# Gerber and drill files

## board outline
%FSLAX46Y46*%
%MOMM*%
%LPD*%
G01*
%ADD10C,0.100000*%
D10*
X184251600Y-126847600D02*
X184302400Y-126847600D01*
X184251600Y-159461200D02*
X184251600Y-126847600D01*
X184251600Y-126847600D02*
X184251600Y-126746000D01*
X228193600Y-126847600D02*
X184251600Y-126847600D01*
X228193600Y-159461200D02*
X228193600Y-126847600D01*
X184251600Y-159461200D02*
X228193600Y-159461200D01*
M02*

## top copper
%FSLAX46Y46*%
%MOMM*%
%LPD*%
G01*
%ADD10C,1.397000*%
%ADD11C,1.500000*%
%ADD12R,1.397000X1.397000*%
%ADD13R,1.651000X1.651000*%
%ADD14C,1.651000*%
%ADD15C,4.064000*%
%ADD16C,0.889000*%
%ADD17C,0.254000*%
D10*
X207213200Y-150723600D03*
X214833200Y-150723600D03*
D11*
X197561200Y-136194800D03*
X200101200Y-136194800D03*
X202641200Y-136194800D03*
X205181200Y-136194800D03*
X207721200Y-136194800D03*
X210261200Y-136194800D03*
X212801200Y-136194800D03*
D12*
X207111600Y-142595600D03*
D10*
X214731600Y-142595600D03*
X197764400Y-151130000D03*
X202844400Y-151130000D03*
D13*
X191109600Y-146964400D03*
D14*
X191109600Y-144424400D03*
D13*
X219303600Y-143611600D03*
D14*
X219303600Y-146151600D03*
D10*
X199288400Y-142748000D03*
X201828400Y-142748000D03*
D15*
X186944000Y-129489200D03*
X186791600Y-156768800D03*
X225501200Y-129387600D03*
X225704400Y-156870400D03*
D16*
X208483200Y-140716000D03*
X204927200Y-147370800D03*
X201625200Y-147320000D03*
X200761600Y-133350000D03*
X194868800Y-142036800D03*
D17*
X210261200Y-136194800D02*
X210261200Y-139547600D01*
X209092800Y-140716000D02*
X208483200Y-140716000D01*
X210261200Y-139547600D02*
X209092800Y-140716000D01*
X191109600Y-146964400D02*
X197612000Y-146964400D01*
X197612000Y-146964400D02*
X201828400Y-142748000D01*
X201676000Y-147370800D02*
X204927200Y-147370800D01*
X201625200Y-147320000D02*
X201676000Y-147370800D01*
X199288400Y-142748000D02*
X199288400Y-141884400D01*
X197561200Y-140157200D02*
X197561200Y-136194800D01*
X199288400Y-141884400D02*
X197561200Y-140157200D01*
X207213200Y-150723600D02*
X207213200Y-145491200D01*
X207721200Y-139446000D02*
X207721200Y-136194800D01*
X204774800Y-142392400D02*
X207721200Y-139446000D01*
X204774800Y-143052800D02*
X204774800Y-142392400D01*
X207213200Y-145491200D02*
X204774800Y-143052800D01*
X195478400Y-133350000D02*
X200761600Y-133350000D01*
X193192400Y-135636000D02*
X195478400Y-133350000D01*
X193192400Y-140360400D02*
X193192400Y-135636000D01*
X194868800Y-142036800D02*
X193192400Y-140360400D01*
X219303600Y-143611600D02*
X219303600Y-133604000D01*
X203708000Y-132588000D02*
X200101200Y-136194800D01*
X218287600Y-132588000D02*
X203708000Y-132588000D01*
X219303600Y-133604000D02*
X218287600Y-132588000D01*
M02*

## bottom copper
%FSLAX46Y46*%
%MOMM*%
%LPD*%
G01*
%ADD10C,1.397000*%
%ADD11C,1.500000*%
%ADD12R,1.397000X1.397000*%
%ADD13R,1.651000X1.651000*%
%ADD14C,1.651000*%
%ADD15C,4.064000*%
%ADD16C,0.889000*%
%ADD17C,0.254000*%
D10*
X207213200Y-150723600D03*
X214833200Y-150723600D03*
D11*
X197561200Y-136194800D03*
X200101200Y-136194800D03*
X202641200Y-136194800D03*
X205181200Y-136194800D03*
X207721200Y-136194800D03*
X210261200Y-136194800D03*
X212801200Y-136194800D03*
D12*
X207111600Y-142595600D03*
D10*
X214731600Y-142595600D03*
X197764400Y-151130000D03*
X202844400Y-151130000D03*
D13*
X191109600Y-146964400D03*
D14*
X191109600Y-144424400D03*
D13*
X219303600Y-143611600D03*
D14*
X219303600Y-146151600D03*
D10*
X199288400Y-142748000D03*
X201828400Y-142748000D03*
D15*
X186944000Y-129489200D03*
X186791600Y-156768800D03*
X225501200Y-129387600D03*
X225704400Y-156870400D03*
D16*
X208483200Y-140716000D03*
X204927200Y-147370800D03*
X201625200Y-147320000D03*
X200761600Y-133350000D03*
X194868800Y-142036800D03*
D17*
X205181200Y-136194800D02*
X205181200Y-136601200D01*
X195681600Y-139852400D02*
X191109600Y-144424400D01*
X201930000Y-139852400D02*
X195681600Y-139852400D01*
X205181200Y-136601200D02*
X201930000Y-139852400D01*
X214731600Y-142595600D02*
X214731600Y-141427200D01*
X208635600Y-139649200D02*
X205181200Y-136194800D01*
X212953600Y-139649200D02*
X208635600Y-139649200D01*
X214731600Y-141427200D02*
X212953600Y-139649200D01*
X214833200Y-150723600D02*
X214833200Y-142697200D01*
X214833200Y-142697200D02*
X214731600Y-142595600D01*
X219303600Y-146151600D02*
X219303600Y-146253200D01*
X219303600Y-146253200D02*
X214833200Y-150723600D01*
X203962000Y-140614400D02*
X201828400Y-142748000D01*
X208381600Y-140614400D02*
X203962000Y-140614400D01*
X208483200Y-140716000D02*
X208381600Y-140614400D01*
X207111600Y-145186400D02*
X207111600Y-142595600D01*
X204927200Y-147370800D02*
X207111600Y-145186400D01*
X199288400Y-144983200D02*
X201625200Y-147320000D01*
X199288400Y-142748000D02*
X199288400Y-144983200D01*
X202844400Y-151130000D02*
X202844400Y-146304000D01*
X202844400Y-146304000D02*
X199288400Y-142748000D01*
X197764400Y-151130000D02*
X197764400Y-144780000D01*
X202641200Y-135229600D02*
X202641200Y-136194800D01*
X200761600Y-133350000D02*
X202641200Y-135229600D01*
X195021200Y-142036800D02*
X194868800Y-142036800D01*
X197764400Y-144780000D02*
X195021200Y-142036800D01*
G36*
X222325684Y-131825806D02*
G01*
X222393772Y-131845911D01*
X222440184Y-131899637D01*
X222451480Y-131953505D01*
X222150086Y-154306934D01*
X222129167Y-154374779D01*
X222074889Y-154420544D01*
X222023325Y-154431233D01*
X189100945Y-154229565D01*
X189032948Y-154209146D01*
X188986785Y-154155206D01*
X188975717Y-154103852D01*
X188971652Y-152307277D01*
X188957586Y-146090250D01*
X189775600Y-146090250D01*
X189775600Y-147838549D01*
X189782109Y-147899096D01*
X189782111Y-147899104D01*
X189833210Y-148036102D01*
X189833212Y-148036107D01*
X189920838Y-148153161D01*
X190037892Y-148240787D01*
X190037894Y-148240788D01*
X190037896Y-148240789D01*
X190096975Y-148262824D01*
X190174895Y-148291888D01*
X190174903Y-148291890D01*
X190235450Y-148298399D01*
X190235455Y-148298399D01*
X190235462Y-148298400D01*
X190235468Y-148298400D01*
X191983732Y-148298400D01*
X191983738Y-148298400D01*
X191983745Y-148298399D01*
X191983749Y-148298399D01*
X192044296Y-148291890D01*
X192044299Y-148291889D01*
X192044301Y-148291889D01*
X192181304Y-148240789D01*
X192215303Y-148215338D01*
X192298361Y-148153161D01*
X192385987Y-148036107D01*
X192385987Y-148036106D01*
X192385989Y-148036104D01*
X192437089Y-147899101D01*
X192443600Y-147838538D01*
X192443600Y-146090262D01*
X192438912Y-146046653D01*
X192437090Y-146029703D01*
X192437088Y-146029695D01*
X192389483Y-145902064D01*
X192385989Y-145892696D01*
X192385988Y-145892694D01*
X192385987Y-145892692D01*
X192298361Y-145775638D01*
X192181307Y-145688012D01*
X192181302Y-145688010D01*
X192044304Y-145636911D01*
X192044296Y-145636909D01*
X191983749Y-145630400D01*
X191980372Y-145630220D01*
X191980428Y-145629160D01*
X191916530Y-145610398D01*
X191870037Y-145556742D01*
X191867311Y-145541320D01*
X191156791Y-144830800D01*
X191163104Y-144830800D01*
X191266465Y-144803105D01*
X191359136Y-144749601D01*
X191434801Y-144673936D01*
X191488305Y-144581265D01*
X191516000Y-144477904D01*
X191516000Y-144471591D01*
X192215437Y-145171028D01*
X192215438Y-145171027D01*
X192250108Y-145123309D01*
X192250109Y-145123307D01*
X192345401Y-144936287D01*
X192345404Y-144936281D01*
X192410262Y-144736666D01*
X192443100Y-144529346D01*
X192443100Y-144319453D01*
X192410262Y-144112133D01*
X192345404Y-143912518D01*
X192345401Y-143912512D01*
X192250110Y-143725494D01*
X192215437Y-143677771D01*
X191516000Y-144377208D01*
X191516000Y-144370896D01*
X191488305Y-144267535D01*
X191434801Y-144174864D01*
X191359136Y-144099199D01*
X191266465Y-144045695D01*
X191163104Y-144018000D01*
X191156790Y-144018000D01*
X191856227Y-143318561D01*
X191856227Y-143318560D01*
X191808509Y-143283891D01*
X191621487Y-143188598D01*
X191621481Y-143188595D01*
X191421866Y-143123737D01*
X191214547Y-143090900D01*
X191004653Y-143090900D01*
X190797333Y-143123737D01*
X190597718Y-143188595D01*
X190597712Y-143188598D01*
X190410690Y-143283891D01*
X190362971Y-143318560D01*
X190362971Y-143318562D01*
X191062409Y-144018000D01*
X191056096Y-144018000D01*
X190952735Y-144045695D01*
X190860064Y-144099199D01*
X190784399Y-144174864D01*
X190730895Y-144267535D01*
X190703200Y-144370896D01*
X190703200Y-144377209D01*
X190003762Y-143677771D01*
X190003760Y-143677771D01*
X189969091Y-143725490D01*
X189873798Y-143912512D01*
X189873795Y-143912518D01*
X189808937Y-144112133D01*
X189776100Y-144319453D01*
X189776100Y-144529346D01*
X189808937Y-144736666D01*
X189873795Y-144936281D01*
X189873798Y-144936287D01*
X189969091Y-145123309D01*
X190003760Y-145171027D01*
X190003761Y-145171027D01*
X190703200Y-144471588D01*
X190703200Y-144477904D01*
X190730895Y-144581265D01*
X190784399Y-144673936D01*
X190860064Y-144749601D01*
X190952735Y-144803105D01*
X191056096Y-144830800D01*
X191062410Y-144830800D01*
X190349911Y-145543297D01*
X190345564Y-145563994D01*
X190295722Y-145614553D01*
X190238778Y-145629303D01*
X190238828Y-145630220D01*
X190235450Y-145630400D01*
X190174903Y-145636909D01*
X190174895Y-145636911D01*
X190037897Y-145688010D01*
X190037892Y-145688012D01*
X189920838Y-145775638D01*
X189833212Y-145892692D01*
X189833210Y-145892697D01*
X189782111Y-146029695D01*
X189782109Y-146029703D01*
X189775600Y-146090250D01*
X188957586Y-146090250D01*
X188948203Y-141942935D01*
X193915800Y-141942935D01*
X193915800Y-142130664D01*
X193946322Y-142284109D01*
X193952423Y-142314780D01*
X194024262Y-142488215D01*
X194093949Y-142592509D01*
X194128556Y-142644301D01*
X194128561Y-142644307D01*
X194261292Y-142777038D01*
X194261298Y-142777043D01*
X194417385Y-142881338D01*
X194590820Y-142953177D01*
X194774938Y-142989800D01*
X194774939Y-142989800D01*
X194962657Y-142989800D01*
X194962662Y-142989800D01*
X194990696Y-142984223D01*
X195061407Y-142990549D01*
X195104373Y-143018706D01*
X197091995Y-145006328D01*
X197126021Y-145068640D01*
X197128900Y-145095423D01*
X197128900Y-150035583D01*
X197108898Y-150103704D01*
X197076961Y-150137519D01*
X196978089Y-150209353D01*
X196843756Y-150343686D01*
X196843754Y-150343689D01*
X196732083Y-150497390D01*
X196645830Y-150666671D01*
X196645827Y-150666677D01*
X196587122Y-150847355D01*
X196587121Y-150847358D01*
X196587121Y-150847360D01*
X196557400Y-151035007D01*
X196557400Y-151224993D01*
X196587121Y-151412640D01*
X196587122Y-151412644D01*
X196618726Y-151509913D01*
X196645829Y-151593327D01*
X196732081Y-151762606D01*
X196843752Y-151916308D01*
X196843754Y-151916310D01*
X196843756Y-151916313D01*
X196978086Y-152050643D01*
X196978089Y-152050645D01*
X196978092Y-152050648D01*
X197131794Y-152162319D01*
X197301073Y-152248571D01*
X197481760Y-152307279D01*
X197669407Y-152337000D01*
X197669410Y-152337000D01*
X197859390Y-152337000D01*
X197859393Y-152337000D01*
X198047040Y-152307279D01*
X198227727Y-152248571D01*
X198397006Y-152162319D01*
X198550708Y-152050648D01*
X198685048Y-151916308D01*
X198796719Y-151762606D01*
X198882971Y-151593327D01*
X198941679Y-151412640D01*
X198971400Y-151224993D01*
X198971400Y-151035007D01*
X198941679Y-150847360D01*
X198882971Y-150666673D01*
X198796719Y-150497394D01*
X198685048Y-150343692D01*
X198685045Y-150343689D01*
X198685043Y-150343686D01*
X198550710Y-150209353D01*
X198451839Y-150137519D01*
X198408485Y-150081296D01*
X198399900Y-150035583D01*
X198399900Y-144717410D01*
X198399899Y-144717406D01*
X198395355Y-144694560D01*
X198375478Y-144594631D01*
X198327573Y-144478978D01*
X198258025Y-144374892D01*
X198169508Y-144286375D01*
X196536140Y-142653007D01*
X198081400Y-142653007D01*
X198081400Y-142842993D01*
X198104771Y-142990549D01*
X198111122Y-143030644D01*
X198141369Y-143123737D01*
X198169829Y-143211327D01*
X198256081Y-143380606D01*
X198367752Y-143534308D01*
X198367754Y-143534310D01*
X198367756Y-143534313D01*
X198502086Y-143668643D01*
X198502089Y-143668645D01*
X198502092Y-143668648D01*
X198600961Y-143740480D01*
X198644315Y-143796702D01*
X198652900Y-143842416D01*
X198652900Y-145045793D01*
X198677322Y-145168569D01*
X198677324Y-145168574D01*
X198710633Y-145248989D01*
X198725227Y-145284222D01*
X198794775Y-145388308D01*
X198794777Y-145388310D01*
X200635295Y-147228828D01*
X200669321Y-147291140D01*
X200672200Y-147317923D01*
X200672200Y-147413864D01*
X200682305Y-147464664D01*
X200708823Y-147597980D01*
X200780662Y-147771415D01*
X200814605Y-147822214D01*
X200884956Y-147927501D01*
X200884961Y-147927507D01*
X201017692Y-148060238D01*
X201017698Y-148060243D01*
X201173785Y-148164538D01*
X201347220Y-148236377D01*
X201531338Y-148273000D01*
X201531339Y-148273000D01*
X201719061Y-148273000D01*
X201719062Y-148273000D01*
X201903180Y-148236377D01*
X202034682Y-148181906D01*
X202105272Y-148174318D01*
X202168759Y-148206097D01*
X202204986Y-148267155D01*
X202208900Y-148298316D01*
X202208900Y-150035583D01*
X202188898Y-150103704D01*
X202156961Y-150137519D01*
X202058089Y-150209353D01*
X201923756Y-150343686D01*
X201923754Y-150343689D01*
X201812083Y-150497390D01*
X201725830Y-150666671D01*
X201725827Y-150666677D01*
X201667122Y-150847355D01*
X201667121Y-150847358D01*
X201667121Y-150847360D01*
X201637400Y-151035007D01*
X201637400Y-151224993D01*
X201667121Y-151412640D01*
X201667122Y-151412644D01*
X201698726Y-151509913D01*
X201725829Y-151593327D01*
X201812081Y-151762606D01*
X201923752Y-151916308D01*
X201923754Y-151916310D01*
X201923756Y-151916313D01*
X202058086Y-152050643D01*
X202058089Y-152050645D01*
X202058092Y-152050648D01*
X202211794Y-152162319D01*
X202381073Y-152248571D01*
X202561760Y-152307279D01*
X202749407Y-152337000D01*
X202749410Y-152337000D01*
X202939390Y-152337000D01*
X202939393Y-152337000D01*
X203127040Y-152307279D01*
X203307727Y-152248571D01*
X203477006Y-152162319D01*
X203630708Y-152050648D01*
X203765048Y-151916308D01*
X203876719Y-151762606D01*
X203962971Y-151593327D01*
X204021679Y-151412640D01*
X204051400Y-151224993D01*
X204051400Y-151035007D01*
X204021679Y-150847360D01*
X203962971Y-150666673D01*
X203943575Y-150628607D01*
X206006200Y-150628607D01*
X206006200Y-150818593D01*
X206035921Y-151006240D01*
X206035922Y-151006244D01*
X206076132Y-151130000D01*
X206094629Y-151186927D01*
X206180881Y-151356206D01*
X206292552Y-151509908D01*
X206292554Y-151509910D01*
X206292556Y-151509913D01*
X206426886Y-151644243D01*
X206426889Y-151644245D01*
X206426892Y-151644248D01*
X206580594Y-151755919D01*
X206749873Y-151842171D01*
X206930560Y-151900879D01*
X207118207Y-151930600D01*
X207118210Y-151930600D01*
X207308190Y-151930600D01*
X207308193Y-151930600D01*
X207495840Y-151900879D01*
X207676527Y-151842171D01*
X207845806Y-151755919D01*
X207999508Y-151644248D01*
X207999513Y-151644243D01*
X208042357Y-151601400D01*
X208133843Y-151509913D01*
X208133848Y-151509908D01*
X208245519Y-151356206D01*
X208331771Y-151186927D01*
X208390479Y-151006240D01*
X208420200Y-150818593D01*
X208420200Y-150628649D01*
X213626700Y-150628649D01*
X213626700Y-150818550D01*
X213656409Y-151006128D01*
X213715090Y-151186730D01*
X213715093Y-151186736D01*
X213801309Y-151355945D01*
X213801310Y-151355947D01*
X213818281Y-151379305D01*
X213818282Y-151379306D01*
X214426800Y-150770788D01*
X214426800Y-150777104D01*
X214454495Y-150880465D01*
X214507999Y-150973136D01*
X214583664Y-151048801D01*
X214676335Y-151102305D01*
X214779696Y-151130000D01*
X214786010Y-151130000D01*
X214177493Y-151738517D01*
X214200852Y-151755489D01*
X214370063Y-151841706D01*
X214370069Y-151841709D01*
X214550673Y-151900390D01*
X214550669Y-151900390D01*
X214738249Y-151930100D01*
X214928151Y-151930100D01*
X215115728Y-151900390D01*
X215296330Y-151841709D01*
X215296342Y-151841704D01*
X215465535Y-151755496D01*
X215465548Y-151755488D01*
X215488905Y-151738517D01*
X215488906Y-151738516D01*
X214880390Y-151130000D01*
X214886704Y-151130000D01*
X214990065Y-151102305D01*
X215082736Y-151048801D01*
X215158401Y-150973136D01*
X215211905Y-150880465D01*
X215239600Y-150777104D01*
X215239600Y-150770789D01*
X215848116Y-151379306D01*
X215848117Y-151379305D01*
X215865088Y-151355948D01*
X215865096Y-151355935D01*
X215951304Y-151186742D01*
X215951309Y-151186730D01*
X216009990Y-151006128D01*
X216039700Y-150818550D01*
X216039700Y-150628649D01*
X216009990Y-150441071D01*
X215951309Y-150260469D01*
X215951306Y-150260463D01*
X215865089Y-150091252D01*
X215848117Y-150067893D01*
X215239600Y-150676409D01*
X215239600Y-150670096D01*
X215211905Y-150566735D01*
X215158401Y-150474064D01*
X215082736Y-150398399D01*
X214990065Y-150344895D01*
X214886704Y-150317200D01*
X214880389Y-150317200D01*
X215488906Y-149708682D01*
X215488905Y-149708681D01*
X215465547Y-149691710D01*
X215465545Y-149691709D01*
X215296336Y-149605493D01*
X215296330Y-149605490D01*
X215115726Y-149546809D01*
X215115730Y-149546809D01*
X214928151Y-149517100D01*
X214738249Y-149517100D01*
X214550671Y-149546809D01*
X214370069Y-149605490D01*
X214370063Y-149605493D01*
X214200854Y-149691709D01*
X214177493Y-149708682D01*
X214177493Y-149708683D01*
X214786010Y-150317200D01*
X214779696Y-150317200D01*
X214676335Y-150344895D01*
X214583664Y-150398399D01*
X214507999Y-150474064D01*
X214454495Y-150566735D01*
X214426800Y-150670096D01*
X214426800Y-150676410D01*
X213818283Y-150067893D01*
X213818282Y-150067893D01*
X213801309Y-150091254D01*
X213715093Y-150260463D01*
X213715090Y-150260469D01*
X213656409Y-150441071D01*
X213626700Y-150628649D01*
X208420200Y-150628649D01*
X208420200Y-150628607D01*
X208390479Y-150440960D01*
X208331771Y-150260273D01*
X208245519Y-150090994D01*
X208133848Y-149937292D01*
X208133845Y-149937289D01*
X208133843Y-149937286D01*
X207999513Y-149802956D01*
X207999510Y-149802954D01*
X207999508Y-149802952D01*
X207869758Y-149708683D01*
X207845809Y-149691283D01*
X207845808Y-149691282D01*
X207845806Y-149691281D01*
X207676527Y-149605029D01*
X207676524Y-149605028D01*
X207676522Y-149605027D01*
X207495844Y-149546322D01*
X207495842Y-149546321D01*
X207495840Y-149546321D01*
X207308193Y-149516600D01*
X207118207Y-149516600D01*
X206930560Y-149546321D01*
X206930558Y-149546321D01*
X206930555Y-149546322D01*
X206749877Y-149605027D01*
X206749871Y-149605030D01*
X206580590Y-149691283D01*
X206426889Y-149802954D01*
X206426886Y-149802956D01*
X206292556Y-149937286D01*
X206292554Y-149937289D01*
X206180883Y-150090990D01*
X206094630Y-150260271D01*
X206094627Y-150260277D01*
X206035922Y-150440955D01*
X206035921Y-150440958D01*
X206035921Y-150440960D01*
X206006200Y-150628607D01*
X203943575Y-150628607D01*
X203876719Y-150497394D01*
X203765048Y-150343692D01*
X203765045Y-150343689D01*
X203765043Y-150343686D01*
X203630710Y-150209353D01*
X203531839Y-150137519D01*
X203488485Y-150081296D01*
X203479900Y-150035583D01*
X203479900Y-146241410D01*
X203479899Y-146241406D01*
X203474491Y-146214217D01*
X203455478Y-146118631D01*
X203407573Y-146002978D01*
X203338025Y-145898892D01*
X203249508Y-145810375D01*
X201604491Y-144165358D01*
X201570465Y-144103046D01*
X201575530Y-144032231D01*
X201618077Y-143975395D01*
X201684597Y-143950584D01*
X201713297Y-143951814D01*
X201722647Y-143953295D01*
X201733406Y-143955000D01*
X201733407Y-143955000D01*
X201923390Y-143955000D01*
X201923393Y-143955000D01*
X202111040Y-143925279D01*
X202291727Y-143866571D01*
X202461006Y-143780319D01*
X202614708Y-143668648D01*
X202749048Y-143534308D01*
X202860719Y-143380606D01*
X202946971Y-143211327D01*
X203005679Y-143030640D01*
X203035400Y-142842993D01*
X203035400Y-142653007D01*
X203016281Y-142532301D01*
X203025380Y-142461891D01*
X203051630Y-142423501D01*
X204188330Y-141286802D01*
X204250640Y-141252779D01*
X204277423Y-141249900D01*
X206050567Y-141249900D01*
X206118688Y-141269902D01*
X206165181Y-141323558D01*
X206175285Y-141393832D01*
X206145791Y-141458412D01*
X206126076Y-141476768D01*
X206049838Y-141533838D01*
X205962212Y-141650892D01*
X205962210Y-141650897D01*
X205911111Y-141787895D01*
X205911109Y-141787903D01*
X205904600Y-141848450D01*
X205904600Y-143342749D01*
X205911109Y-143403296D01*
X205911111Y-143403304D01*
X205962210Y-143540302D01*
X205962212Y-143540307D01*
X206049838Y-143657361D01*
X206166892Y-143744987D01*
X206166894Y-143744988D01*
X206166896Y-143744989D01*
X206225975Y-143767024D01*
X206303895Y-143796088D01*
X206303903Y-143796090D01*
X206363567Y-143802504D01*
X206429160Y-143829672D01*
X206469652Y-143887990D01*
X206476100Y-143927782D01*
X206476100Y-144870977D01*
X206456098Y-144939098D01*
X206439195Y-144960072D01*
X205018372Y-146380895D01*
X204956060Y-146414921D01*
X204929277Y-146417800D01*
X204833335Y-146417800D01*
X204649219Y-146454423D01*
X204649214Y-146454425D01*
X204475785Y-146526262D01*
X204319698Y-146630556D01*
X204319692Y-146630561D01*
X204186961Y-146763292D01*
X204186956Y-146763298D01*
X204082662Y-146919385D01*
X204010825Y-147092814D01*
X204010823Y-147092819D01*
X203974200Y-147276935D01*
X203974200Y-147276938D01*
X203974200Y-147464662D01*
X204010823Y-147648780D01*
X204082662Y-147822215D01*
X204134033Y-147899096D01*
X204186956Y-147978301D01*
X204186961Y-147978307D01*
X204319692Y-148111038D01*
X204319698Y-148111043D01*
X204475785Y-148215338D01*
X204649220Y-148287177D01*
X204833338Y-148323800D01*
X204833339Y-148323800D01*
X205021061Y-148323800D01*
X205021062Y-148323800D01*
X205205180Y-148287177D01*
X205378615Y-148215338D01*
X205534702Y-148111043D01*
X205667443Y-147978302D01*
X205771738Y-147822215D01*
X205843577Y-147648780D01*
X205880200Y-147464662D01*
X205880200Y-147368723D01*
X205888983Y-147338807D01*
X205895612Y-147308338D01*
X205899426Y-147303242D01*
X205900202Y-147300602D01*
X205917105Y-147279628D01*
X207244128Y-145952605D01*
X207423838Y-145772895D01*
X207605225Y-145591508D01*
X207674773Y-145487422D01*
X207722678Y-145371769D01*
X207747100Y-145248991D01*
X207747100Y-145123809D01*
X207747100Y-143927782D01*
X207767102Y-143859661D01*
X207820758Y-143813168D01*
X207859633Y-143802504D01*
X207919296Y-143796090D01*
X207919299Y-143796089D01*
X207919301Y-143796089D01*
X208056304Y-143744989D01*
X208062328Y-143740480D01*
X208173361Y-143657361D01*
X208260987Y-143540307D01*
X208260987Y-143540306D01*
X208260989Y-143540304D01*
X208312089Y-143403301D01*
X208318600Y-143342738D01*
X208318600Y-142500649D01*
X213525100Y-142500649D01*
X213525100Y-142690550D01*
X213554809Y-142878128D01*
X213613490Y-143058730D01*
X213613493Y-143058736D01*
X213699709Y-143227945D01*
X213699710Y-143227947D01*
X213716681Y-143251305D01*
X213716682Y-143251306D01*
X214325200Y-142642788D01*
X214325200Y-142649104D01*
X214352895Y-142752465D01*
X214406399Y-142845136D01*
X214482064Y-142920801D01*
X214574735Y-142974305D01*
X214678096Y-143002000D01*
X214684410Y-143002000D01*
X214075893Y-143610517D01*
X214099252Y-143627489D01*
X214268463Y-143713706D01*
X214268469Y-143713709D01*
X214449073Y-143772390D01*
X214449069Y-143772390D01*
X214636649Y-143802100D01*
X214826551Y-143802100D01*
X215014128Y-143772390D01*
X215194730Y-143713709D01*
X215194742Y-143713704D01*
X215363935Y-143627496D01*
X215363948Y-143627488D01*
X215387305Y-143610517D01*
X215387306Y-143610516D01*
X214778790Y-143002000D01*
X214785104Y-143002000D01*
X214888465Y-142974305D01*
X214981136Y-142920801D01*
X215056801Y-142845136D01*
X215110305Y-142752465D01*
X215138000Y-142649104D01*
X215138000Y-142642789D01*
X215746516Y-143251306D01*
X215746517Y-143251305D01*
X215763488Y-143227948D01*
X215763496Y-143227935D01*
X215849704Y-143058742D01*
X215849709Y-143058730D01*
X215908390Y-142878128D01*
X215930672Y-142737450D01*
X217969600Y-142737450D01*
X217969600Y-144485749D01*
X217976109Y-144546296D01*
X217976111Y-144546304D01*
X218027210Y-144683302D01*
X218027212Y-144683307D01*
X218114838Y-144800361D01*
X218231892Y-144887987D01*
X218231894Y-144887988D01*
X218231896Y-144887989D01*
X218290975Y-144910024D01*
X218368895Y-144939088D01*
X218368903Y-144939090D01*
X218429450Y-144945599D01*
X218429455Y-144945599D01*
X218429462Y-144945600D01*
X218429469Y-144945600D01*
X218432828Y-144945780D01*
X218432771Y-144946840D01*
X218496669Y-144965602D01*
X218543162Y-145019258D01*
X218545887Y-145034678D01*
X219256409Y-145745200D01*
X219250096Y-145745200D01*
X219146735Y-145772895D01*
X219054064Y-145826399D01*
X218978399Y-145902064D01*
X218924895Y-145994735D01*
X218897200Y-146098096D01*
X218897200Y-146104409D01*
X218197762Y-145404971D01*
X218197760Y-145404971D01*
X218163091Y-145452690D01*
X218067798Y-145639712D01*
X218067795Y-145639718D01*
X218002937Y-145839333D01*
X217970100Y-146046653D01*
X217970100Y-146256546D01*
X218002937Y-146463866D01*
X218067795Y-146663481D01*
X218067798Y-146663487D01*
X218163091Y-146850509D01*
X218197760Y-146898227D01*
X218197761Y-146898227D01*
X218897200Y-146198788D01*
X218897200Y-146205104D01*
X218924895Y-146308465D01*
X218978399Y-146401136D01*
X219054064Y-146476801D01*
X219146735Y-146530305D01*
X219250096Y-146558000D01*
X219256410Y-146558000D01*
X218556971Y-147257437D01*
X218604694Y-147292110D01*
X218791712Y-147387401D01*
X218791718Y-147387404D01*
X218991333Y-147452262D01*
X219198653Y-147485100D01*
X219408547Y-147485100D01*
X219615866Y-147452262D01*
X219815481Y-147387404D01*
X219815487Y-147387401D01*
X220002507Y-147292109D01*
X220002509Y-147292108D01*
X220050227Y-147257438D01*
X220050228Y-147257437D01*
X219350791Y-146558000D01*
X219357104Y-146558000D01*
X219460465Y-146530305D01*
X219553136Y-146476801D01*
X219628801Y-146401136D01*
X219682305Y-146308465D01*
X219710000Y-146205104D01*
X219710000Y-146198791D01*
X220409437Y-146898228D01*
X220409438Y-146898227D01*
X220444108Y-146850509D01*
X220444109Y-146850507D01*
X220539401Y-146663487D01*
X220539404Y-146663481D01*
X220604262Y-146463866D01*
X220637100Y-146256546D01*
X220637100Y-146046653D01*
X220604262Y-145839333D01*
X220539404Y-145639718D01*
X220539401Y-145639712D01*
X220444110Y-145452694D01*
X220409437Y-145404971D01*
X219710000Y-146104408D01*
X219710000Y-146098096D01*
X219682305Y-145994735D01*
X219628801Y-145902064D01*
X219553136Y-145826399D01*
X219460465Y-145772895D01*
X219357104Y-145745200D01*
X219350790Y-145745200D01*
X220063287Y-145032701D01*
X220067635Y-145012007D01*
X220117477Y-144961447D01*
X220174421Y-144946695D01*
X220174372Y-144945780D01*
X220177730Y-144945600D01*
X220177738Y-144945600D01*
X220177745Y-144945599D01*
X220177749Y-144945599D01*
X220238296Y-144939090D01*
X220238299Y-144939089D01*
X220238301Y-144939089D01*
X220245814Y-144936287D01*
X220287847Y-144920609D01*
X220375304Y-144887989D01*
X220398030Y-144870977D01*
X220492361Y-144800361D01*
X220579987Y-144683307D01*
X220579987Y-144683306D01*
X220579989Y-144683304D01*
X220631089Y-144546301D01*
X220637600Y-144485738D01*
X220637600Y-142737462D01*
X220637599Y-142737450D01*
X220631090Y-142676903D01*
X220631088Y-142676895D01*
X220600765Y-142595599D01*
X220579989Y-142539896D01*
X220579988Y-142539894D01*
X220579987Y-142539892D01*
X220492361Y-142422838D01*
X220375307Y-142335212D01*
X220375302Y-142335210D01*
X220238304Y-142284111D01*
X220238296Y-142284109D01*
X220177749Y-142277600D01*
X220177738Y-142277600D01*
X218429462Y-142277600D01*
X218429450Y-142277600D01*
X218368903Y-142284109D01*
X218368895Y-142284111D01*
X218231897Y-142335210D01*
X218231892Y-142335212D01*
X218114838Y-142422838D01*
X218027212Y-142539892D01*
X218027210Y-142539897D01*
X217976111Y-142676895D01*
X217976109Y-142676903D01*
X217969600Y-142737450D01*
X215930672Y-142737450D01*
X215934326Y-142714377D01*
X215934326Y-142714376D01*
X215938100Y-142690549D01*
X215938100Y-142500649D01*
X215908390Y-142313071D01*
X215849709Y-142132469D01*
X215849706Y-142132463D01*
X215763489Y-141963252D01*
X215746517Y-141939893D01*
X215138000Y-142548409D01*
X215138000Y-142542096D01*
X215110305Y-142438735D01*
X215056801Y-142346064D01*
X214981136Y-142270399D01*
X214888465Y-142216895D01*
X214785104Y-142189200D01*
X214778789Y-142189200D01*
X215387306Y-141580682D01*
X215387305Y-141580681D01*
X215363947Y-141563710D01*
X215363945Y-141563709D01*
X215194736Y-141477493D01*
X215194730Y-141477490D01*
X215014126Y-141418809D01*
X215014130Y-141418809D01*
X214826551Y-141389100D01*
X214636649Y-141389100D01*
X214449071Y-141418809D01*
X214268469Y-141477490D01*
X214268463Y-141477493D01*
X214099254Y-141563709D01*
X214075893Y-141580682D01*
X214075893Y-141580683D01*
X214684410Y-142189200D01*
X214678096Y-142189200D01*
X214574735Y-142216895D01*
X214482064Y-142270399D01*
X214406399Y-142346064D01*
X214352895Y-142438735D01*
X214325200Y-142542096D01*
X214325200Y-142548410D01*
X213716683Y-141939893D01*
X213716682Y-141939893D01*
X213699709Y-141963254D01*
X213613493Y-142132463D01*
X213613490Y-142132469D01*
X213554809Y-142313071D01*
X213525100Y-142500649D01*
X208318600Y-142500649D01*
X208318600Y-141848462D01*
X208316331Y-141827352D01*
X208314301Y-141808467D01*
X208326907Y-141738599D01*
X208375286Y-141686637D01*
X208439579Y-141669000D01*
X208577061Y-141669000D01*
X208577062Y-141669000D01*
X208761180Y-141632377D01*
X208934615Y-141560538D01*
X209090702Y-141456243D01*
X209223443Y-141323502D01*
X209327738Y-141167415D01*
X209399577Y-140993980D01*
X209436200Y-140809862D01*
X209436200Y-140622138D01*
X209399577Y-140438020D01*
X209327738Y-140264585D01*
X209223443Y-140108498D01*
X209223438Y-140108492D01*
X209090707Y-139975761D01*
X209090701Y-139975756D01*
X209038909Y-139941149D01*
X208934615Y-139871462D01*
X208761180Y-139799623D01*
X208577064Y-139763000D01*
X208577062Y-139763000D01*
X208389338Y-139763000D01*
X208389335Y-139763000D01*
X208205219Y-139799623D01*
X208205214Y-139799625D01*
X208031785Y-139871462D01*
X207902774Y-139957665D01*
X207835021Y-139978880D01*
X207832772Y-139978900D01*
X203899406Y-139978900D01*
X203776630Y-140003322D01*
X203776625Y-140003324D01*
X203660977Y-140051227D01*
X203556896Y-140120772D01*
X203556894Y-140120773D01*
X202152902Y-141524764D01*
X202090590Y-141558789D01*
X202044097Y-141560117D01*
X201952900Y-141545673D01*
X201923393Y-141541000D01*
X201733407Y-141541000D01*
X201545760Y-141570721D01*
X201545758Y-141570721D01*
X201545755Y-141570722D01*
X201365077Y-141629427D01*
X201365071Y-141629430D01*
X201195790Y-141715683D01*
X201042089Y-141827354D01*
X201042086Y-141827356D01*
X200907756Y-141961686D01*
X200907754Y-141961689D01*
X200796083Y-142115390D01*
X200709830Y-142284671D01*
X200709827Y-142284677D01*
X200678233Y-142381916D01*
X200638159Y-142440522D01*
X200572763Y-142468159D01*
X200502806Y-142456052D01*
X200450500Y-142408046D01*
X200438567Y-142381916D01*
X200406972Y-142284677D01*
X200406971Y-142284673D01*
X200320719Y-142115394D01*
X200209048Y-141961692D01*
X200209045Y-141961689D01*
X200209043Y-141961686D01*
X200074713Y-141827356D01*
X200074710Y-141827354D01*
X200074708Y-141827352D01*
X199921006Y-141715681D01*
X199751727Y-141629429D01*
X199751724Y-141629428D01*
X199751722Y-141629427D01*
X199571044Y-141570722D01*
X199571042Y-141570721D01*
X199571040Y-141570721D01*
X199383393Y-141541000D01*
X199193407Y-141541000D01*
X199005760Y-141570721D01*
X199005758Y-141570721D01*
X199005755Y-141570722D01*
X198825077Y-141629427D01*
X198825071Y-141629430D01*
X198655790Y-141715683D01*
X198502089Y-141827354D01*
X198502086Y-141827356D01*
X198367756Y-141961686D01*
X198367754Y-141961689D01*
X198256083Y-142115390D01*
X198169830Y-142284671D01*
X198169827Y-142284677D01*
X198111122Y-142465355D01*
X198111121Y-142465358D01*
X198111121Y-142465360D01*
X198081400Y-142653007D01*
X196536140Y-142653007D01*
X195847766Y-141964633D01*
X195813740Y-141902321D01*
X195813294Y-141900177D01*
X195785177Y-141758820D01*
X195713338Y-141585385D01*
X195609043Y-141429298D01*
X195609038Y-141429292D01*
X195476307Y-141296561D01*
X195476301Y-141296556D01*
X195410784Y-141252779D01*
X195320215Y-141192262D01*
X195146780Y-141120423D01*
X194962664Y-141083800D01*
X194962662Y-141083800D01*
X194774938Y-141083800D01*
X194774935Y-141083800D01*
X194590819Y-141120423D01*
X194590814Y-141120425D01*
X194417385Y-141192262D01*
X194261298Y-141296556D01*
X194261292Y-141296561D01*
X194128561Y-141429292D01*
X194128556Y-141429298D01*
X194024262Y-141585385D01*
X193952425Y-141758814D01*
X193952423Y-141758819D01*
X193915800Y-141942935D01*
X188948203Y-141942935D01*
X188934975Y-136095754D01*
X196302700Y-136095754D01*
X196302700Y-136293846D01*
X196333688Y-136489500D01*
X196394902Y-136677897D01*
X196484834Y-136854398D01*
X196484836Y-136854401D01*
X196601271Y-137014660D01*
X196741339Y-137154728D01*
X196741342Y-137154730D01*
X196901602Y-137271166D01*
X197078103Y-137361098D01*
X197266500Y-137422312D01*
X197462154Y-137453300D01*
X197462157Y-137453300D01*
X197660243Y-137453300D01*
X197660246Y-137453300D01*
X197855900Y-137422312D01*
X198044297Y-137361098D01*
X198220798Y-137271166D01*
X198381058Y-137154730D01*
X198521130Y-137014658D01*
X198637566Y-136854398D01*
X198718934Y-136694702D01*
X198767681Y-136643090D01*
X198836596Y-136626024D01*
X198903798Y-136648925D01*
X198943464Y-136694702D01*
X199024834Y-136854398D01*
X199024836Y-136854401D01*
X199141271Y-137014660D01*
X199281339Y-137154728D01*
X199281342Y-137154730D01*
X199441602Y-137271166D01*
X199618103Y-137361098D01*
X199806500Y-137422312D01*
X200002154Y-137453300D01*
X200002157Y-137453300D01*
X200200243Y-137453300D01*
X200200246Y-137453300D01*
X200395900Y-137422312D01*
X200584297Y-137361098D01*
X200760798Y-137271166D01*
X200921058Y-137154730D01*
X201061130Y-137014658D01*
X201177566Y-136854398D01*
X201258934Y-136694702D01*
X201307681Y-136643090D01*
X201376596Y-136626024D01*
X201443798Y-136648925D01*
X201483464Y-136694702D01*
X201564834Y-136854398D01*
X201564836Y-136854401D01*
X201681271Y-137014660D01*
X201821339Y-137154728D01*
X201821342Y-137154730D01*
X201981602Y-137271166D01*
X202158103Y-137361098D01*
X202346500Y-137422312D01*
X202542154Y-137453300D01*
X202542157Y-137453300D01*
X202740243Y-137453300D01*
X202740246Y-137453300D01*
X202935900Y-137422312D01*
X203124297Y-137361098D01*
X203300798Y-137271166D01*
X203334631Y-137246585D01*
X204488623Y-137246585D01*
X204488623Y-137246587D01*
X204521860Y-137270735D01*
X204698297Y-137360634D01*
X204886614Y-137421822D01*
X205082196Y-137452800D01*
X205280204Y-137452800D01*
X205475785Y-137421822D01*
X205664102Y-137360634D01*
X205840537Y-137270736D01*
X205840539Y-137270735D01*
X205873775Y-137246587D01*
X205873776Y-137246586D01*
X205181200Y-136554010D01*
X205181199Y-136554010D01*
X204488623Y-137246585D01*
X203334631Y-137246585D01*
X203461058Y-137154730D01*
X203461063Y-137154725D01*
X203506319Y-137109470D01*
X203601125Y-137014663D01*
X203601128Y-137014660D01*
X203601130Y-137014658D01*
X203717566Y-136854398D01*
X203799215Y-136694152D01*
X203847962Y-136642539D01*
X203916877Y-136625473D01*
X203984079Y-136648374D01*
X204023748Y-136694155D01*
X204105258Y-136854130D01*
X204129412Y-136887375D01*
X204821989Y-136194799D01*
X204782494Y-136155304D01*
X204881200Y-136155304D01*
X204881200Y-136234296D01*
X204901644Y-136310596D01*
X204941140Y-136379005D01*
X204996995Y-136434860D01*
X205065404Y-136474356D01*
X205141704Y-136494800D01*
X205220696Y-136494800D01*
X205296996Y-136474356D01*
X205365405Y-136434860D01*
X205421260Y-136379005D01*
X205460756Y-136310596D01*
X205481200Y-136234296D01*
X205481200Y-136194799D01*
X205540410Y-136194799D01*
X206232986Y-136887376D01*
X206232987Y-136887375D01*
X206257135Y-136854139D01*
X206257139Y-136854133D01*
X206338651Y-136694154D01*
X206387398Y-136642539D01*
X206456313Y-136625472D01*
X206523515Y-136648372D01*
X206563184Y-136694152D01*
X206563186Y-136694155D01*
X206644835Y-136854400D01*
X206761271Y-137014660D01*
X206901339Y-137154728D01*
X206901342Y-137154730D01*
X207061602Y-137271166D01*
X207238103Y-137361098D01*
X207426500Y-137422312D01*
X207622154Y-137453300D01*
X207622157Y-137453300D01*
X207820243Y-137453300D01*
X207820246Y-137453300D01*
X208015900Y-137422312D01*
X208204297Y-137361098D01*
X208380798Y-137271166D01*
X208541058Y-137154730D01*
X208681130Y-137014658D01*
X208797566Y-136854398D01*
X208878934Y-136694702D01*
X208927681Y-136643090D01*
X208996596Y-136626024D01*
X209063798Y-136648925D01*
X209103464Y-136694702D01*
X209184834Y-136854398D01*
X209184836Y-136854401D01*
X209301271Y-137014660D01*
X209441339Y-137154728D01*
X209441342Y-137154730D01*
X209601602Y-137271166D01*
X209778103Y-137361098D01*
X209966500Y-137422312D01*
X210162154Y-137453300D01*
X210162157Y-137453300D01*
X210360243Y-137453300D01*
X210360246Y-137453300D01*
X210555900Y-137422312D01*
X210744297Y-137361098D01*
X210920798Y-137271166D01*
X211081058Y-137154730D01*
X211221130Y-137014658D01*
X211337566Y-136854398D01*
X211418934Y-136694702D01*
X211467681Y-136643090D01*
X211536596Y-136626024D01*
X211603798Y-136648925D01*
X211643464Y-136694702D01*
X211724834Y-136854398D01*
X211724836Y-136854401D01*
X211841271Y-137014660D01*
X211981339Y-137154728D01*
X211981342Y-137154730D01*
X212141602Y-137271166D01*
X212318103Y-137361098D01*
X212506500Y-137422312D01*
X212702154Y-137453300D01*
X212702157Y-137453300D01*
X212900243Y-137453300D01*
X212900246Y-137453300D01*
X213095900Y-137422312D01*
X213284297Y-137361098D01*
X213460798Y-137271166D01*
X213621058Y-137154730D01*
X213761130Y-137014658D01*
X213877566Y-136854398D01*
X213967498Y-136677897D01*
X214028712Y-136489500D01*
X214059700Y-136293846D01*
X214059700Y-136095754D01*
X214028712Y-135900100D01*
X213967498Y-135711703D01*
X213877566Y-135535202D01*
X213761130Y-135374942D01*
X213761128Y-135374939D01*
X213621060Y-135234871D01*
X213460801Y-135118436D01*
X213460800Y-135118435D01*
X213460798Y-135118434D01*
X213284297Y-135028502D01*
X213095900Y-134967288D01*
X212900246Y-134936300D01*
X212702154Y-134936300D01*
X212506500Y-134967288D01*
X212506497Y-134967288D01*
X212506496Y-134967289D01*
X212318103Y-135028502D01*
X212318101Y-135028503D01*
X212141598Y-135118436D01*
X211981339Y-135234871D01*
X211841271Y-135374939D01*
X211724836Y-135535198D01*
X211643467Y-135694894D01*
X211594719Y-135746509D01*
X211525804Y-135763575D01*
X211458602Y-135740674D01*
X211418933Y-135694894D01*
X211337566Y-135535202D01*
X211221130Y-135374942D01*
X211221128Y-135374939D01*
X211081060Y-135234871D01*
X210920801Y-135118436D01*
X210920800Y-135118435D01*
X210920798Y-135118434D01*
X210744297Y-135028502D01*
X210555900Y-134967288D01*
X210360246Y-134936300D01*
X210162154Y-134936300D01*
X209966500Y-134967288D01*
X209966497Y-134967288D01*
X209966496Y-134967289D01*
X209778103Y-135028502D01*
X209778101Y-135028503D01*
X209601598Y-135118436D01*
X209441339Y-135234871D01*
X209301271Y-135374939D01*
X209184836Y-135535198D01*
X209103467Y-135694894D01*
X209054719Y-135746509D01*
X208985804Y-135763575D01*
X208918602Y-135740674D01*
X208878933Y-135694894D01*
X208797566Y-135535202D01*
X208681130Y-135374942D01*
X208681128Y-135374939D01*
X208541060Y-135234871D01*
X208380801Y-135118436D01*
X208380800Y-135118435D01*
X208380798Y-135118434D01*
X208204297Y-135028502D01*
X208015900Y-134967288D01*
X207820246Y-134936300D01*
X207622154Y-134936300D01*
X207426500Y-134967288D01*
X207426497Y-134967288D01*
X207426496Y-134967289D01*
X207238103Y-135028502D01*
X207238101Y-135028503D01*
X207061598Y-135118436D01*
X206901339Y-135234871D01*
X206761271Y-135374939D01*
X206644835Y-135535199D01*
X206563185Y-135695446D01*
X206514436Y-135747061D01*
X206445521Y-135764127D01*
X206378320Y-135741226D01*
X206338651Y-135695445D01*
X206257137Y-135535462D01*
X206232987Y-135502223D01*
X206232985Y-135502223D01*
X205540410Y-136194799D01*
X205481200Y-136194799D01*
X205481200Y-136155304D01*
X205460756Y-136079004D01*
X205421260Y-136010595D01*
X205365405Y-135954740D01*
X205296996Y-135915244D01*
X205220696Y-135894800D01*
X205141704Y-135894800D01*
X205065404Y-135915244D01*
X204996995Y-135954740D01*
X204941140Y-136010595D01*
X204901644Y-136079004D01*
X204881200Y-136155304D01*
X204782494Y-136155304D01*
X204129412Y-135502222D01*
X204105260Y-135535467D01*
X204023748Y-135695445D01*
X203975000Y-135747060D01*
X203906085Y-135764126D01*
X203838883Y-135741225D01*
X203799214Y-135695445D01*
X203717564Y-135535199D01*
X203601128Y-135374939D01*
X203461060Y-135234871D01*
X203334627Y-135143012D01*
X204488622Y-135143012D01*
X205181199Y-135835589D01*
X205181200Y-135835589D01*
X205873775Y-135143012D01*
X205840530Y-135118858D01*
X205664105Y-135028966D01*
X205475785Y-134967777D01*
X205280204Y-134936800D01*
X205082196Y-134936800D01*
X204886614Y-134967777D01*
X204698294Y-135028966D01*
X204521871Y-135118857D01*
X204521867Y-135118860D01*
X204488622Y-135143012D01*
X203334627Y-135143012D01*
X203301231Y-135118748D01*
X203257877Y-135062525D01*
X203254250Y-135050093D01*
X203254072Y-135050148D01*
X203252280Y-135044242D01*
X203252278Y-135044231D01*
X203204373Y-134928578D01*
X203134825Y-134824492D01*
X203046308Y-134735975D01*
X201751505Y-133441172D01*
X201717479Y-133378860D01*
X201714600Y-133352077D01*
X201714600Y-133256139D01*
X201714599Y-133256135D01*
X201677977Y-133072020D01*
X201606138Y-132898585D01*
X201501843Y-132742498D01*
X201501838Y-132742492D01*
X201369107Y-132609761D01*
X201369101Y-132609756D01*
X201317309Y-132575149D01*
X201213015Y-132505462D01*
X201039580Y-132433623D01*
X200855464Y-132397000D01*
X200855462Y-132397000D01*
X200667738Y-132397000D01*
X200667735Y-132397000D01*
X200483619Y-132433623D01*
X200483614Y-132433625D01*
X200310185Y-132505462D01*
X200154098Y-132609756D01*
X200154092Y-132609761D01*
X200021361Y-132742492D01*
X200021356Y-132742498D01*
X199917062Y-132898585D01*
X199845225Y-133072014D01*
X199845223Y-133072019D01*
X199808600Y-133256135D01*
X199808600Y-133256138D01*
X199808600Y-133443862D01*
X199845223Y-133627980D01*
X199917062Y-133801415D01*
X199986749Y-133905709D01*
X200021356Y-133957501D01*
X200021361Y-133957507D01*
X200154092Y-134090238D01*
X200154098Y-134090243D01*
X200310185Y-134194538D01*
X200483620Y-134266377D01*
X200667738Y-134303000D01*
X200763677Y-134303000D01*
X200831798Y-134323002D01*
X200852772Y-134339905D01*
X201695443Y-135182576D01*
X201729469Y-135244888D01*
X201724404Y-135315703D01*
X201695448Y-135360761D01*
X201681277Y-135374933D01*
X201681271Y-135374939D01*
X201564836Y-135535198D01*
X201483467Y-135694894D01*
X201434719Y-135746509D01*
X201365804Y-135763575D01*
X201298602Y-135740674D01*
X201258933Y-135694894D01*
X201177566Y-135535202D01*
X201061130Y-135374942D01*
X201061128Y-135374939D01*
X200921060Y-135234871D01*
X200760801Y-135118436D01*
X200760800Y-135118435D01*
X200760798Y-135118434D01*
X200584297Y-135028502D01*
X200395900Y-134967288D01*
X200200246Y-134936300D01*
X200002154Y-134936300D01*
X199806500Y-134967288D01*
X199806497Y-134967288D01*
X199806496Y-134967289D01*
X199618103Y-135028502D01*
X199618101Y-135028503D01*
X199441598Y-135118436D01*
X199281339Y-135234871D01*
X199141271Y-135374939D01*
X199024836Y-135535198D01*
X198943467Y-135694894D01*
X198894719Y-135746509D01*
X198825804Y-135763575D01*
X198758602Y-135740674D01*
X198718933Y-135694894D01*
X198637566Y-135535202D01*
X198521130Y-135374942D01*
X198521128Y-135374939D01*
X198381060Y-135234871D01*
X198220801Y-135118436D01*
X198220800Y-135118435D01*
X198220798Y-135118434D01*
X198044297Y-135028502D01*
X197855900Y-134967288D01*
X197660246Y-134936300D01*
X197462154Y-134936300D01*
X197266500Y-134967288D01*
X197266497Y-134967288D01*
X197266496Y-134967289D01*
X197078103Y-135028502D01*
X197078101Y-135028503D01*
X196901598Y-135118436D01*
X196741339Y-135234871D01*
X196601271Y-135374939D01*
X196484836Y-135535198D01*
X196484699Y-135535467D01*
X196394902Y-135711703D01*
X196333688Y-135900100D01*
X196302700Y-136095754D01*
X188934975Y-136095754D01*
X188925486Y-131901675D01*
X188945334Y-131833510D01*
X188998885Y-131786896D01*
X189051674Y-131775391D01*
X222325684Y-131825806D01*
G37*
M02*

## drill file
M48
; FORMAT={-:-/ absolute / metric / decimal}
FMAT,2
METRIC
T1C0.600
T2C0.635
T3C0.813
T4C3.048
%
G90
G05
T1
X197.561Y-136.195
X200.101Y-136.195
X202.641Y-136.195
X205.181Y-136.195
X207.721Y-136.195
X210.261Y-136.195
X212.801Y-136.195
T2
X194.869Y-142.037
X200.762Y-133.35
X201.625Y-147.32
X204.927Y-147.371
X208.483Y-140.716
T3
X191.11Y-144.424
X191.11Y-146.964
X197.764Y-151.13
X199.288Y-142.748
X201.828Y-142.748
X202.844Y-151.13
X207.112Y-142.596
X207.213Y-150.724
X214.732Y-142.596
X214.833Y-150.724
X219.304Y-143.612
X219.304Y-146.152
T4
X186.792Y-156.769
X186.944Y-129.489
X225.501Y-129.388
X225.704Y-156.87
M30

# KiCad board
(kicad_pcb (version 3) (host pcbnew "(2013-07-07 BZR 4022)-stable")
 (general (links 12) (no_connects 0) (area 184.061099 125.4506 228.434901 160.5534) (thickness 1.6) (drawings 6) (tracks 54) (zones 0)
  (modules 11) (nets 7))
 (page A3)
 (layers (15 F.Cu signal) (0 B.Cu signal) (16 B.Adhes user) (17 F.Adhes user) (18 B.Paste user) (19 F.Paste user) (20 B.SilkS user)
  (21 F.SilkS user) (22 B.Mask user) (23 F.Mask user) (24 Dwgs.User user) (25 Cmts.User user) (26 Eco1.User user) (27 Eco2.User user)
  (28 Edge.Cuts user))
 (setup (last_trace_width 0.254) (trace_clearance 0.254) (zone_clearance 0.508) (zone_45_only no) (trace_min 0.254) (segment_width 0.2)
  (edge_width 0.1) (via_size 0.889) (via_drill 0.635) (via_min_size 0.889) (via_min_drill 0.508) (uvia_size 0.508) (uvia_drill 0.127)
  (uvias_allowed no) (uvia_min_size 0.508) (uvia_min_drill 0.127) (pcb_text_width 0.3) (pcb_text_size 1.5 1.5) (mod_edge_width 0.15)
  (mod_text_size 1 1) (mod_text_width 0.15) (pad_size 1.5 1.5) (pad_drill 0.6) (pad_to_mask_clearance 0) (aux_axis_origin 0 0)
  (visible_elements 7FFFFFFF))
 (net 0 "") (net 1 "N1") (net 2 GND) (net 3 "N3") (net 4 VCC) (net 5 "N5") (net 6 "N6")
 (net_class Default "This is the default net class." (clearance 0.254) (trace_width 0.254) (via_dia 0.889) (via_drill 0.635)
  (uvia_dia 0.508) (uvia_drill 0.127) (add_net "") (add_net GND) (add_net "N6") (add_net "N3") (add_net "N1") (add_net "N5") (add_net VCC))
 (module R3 (layer F.Cu) (at 211.0232 150.7236) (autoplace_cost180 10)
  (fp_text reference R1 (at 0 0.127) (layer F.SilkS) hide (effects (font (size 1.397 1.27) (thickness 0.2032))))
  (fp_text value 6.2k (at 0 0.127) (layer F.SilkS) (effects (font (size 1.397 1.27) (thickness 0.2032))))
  (pad 1 thru_hole circle (at -3.81 0) (size 1.397 1.397) (drill 0.8128) (layers *.Cu *.Mask F.SilkS) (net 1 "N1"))
  (pad 2 thru_hole circle (at 3.81 0) (size 1.397 1.397) (drill 0.8128) (layers *.Cu *.Mask F.SilkS) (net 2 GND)))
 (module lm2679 (layer F.Cu) (at 205.1812 137.4648)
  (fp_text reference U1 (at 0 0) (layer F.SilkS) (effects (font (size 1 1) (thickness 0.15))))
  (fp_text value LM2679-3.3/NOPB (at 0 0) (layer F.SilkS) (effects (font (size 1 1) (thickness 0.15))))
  (pad 1 thru_hole circle (at -7.62 -1.27) (size 1.5 1.5) (drill 0.6) (layers *.Cu *.Mask F.SilkS) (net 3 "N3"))
  (pad 2 thru_hole circle (at -5.08 -1.27) (size 1.5 1.5) (drill 0.6) (layers *.Cu *.Mask F.SilkS) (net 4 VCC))
  (pad 3 thru_hole circle (at -2.54 -1.27) (size 1.5 1.5) (drill 0.6) (layers *.Cu *.Mask F.SilkS) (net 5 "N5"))
  (pad 4 thru_hole circle (at 0 -1.27) (size 1.5 1.5) (drill 0.6) (layers *.Cu *.Mask F.SilkS) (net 2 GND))
  (pad 5 thru_hole circle (at 2.54 -1.27) (size 1.5 1.5) (drill 0.6) (layers *.Cu *.Mask F.SilkS) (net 1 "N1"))
  (pad 6 thru_hole circle (at 5.08 -1.27) (size 1.5 1.5) (drill 0.6) (layers *.Cu *.Mask F.SilkS) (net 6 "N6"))
  (pad 7 thru_hole circle (at 7.62 -1.27) (size 1.5 1.5) (drill 0.6) (layers *.Cu *.Mask F.SilkS)))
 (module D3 (layer F.Cu) (at 210.9216 142.5956 180)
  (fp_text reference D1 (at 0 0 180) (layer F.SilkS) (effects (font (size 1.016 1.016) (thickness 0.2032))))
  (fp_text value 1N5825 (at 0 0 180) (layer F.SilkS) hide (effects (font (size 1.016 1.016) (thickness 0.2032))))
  (pad 2 thru_hole rect (at 3.81 0 180) (size 1.397 1.397) (drill 0.8128) (layers *.Cu *.Mask F.SilkS) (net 3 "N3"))
  (pad 1 thru_hole circle (at -3.81 0 180) (size 1.397 1.397) (drill 0.8128) (layers *.Cu *.Mask F.SilkS) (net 2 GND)))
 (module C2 (layer F.Cu) (at 200.3044 151.13)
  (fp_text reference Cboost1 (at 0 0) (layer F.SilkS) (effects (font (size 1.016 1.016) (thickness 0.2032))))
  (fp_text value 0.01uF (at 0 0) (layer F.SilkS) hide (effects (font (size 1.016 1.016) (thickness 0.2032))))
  (pad 1 thru_hole circle (at -2.54 0) (size 1.397 1.397) (drill 0.8128) (layers *.Cu *.Mask F.SilkS) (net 5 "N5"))
  (pad 2 thru_hole circle (at 2.54 0) (size 1.397 1.397) (drill 0.8128) (layers *.Cu *.Mask F.SilkS) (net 3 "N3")))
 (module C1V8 (layer F.Cu) (at 191.1096 145.6944 90)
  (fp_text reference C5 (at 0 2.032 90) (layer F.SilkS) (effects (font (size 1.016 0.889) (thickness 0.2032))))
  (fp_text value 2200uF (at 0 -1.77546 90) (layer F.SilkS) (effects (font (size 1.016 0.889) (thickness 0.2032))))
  (pad 1 thru_hole rect (at -1.27 0 90) (size 1.651 1.651) (drill 0.8128) (layers *.Cu *.Mask F.SilkS) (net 6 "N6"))
  (pad 2 thru_hole circle (at 1.27 0 90) (size 1.651 1.651) (drill 0.8128) (layers *.Cu *.Mask F.SilkS) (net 2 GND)))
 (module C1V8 (layer F.Cu) (at 219.3036 144.8816 270)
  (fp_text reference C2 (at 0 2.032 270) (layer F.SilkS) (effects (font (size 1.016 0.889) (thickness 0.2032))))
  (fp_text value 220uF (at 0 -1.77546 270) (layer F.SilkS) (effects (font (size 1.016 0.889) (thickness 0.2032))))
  (pad 1 thru_hole rect (at -1.27 0 270) (size 1.651 1.651) (drill 0.8128) (layers *.Cu *.Mask F.SilkS) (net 4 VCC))
  (pad 2 thru_hole circle (at 1.27 0 270) (size 1.651 1.651) (drill 0.8128) (layers *.Cu *.Mask F.SilkS) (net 2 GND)))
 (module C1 (layer F.Cu) (at 200.5584 142.748)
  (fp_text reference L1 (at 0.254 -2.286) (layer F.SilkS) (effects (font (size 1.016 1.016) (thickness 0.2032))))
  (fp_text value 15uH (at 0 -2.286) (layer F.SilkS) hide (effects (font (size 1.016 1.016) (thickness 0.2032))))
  (pad 1 thru_hole circle (at -1.27 0) (size 1.397 1.397) (drill 0.8128) (layers *.Cu *.Mask F.SilkS) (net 3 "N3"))
  (pad 2 thru_hole circle (at 1.27 0) (size 1.397 1.397) (drill 0.8128) (layers *.Cu *.Mask F.SilkS) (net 6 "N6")))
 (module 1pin (layer F.Cu) (at 186.944 129.4892)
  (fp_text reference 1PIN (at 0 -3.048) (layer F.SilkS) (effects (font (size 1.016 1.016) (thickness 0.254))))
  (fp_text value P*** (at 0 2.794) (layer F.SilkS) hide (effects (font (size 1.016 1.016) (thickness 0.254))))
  (pad 1 thru_hole circle (at 0 0) (size 4.064 4.064) (drill 3.048) (layers *.Cu *.Mask F.SilkS)))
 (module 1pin (layer F.Cu) (at 186.7916 156.7688)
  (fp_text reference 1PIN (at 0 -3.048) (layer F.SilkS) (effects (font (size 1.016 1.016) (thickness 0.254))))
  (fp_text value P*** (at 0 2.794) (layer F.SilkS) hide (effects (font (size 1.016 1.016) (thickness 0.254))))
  (pad 1 thru_hole circle (at 0 0) (size 4.064 4.064) (drill 3.048) (layers *.Cu *.Mask F.SilkS)))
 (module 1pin (layer F.Cu) (at 225.5012 129.3876)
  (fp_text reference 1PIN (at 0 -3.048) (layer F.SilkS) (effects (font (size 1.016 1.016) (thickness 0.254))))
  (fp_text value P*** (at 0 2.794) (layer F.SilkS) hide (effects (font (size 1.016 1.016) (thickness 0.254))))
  (pad 1 thru_hole circle (at 0 0) (size 4.064 4.064) (drill 3.048) (layers *.Cu *.Mask F.SilkS)))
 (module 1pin (layer F.Cu) (at 225.7044 156.8704)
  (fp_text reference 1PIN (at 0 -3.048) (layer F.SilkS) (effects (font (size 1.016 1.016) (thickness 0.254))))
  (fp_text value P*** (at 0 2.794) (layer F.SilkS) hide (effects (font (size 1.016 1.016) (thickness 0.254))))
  (pad 1 thru_hole circle (at 0 0) (size 4.064 4.064) (drill 3.048) (layers *.Cu *.Mask F.SilkS)))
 (gr_line (start 184.2516 126.8476) (end 184.3024 126.8476) (angle 90) (layer Edge.Cuts) (width 0.1))
 (gr_line (start 184.2516 159.4612) (end 184.2516 126.8476) (angle 90) (layer Edge.Cuts) (width 0.1))
 (gr_line (start 184.2516 126.8476) (end 184.2516 126.746) (angle 90) (layer Edge.Cuts) (width 0.1))
 (gr_line (start 228.1936 126.8476) (end 184.2516 126.8476) (angle 90) (layer Edge.Cuts) (width 0.1))
 (gr_line (start 228.1936 159.4612) (end 228.1936 126.8476) (angle 90) (layer Edge.Cuts) (width 0.1))
 (gr_line (start 184.2516 159.4612) (end 228.1936 159.4612) (angle 90) (layer Edge.Cuts) (width 0.1))
 (segment (start 205.1812 136.1948) (end 205.1812 136.6012) (width 0.254) (layer B.Cu) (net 2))
 (segment (start 195.6816 139.8524) (end 191.1096 144.4244) (width 0.254) (layer B.Cu) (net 2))
 (segment (start 201.93 139.8524) (end 195.6816 139.8524) (width 0.254) (layer B.Cu) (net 2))
 (segment (start 205.1812 136.6012) (end 201.93 139.8524) (width 0.254) (layer B.Cu) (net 2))
 (segment (start 214.7316 142.5956) (end 214.7316 141.4272) (width 0.254) (layer B.Cu) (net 2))
 (segment (start 208.6356 139.6492) (end 205.1812 136.1948) (width 0.254) (layer B.Cu) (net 2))
 (segment (start 212.9536 139.6492) (end 208.6356 139.6492) (width 0.254) (layer B.Cu) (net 2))
 (segment (start 214.7316 141.4272) (end 212.9536 139.6492) (width 0.254) (layer B.Cu) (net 2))
 (segment (start 214.8332 150.7236) (end 214.8332 142.6972) (width 0.254) (layer B.Cu) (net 2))
 (segment (start 214.8332 142.6972) (end 214.7316 142.5956) (width 0.254) (layer B.Cu) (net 2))
 (segment (start 219.3036 146.1516) (end 219.3036 146.2532) (width 0.254) (layer B.Cu) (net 2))
 (segment (start 219.3036 146.2532) (end 214.8332 150.7236) (width 0.254) (layer B.Cu) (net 2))
 (segment (start 210.2612 136.1948) (end 210.2612 139.5476) (width 0.254) (layer F.Cu) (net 6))
 (segment (start 203.962 140.6144) (end 201.8284 142.748) (width 0.254) (layer B.Cu) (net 6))
 (segment (start 208.3816 140.6144) (end 203.962 140.6144) (width 0.254) (layer B.Cu) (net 6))
 (segment (start 208.4832 140.716) (end 208.3816 140.6144) (width 0.254) (layer B.Cu) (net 6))
 (via (at 208.4832 140.716) (size 0.889) (layers F.Cu B.Cu) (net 6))
 (segment (start 209.0928 140.716) (end 208.4832 140.716) (width 0.254) (layer F.Cu) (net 6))
 (segment (start 210.2612 139.5476) (end 209.0928 140.716) (width 0.254) (layer F.Cu) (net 6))
 (segment (start 191.1096 146.9644) (end 197.612 146.9644) (width 0.254) (layer F.Cu) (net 6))
 (segment (start 197.612 146.9644) (end 201.8284 142.748) (width 0.254) (layer F.Cu) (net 6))
 (segment (start 207.1116 145.1864) (end 207.1116 142.5956) (width 0.254) (layer B.Cu) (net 3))
 (segment (start 204.9272 147.3708) (end 207.1116 145.1864) (width 0.254) (layer B.Cu) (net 3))
 (via (at 204.9272 147.3708) (size 0.889) (layers F.Cu B.Cu) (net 3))
 (segment (start 201.676 147.3708) (end 204.9272 147.3708) (width 0.254) (layer F.Cu) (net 3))
 (segment (start 201.6252 147.32) (end 201.676 147.3708) (width 0.254) (layer F.Cu) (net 3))
 (via (at 201.6252 147.32) (size 0.889) (layers F.Cu B.Cu) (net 3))
 (segment (start 199.2884 144.9832) (end 201.6252 147.32) (width 0.254) (layer B.Cu) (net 3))
 (segment (start 199.2884 142.748) (end 199.2884 144.9832) (width 0.254) (layer B.Cu) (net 3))
 (segment (start 202.8444 151.13) (end 202.8444 146.304) (width 0.254) (layer B.Cu) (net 3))
 (segment (start 202.8444 146.304) (end 199.2884 142.748) (width 0.254) (layer B.Cu) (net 3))
 (segment (start 199.2884 142.748) (end 199.2884 141.8844) (width 0.254) (layer F.Cu) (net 3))
 (segment (start 197.5612 140.1572) (end 197.5612 136.1948) (width 0.254) (layer F.Cu) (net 3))
 (segment (start 199.2884 141.8844) (end 197.5612 140.1572) (width 0.254) (layer F.Cu) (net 3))
 (segment (start 207.2132 150.7236) (end 207.2132 145.4912) (width 0.254) (layer F.Cu) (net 1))
 (segment (start 207.7212 139.446) (end 207.7212 136.1948) (width 0.254) (layer F.Cu) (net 1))
 (segment (start 204.7748 142.3924) (end 207.7212 139.446) (width 0.254) (layer F.Cu) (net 1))
 (segment (start 204.7748 143.0528) (end 204.7748 142.3924) (width 0.254) (layer F.Cu) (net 1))
 (segment (start 207.2132 145.4912) (end 204.7748 143.0528) (width 0.254) (layer F.Cu) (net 1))
 (segment (start 197.7644 151.13) (end 197.7644 144.78) (width 0.254) (layer B.Cu) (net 5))
 (segment (start 202.6412 135.2296) (end 202.6412 136.1948) (width 0.254) (layer B.Cu) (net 5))
 (segment (start 200.7616 133.35) (end 202.6412 135.2296) (width 0.254) (layer B.Cu) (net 5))
 (via (at 200.7616 133.35) (size 0.889) (layers F.Cu B.Cu) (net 5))
 (segment (start 195.4784 133.35) (end 200.7616 133.35) (width 0.254) (layer F.Cu) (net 5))
 (segment (start 193.1924 135.636) (end 195.4784 133.35) (width 0.254) (layer F.Cu) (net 5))
 (segment (start 193.1924 140.3604) (end 193.1924 135.636) (width 0.254) (layer F.Cu) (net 5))
 (segment (start 194.8688 142.0368) (end 193.1924 140.3604) (width 0.254) (layer F.Cu) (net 5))
 (via (at 194.8688 142.0368) (size 0.889) (layers F.Cu B.Cu) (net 5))
 (segment (start 195.0212 142.0368) (end 194.8688 142.0368) (width 0.254) (layer B.Cu) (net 5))
 (segment (start 197.7644 144.78) (end 195.0212 142.0368) (width 0.254) (layer B.Cu) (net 5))
 (segment (start 219.3036 143.6116) (end 219.3036 133.604) (width 0.254) (layer F.Cu) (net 4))
 (segment (start 203.708 132.588) (end 200.1012 136.1948) (width 0.254) (layer F.Cu) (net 4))
 (segment (start 218.2876 132.588) (end 203.708 132.588) (width 0.254) (layer F.Cu) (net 4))
 (segment (start 219.3036 133.604) (end 218.2876 132.588) (width 0.254) (layer F.Cu) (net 4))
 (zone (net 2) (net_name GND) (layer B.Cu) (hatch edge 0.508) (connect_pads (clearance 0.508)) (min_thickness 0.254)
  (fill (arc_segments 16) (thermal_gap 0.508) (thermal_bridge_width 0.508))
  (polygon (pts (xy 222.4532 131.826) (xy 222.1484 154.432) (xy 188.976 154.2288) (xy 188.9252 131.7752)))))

